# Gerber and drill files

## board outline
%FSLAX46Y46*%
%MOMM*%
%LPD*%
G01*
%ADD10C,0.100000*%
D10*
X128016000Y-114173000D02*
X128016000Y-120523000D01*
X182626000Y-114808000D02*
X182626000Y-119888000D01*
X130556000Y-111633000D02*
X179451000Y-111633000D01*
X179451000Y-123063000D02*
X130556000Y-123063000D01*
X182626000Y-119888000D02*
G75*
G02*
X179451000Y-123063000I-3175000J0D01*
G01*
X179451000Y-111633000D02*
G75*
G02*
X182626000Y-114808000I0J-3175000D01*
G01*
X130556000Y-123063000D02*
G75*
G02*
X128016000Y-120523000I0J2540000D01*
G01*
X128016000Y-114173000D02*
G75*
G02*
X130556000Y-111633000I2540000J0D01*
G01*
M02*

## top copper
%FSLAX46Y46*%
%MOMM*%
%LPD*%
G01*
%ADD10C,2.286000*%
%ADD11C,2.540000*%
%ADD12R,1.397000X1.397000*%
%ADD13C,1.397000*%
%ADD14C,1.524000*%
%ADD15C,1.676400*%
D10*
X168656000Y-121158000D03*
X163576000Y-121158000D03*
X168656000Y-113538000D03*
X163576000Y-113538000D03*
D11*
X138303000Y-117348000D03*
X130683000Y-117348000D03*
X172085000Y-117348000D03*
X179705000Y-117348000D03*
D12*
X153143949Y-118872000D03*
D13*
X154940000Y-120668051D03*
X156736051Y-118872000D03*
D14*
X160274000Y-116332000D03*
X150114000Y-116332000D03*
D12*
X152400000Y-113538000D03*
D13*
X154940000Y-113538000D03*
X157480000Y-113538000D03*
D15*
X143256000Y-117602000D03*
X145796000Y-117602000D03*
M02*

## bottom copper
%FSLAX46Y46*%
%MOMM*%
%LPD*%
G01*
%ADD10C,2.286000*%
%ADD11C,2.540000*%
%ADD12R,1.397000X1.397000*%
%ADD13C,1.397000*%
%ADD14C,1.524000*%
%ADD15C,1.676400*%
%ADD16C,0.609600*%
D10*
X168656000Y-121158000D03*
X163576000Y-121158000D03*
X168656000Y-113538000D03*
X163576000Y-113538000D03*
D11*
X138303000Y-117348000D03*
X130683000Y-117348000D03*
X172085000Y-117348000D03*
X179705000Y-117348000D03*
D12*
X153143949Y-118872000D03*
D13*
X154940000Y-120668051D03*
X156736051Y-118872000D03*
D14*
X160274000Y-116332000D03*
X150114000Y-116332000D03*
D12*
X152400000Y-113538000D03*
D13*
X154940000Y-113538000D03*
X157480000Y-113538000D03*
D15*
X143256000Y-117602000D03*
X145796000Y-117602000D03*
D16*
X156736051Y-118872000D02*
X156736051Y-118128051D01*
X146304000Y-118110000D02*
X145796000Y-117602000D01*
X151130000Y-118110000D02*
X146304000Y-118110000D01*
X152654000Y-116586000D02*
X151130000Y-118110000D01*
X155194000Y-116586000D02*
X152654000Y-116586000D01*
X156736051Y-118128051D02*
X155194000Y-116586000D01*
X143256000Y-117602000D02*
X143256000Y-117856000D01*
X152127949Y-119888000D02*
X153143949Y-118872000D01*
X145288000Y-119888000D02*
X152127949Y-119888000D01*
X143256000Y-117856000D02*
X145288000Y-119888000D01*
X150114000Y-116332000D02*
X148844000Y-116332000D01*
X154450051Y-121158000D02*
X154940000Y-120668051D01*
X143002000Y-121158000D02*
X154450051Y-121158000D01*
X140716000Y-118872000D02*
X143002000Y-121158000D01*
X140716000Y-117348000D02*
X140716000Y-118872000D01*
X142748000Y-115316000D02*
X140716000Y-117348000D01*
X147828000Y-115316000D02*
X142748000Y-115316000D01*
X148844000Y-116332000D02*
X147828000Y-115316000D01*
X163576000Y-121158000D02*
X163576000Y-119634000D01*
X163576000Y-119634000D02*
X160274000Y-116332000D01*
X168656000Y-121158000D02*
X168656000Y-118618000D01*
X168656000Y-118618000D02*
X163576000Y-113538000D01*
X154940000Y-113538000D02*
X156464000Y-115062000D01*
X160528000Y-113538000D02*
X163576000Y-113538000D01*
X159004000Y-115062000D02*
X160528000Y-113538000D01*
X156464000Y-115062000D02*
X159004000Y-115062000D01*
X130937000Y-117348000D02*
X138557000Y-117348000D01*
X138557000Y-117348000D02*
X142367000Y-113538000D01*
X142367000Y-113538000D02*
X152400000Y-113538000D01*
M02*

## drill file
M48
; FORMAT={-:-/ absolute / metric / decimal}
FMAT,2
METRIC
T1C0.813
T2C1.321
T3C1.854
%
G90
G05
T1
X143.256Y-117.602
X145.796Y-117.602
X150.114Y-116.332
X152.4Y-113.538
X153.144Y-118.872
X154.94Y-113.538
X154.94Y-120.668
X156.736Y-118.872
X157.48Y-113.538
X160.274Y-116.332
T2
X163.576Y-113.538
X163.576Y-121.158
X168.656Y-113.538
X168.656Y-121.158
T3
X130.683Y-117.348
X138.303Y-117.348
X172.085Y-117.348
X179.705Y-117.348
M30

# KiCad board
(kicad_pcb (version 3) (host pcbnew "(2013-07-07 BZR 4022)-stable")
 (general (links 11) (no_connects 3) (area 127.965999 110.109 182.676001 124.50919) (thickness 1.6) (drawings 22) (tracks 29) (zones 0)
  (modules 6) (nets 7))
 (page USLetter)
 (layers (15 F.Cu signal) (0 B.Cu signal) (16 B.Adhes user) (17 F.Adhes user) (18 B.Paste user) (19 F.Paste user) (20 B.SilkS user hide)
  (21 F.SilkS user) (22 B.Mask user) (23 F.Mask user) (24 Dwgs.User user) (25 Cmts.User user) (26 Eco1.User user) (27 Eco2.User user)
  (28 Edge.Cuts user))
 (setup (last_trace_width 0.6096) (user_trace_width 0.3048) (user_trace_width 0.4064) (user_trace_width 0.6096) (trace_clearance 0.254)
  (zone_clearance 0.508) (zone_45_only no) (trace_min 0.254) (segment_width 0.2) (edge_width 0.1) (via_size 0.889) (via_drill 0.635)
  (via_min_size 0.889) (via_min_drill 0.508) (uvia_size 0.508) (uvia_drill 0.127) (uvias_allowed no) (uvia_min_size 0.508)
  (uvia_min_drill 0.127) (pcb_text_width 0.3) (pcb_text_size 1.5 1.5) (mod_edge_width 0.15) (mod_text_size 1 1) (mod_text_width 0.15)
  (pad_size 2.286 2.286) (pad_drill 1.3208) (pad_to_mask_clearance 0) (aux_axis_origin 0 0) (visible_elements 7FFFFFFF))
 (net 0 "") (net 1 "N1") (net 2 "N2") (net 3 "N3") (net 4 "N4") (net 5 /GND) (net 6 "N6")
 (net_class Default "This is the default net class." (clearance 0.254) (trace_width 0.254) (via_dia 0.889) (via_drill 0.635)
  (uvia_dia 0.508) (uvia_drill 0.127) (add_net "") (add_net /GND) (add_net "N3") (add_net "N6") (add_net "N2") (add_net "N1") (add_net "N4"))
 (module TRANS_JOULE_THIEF (layer F.Cu) (at 166.116 118.618 180)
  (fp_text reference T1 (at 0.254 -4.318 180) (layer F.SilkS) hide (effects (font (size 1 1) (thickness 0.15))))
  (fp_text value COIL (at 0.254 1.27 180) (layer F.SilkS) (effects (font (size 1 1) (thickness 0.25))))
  (pad 1 thru_hole circle (at -2.54 -2.54 180) (size 2.286 2.286) (drill 1.3208) (layers *.Cu *.Mask F.SilkS) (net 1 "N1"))
  (pad 2 thru_hole circle (at 2.54 -2.54 180) (size 2.286 2.286) (drill 1.3208) (layers *.Cu *.Mask F.SilkS) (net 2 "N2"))
  (pad 3 thru_hole circle (at -2.54 5.08 180) (size 2.286 2.286) (drill 1.3208) (layers *.Cu *.Mask F.SilkS) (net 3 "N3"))
  (pad 4 thru_hole circle (at 2.54 5.08 180) (size 2.286 2.286) (drill 1.3208) (layers *.Cu *.Mask F.SilkS) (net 1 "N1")))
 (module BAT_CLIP (layer F.Cu) (at 155.321 117.348)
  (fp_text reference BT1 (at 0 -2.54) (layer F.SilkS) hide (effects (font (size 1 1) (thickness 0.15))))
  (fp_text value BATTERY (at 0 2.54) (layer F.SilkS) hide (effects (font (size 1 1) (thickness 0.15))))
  (pad 1 thru_hole circle (at -17.018 0) (size 2.54 2.54) (drill 1.8542) (layers *.Cu *.Mask F.SilkS) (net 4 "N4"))
  (pad 1 thru_hole circle (at -24.638 0) (size 2.54 2.54) (drill 1.8542) (layers *.Cu *.Mask F.SilkS) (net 4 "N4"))
  (pad 2 thru_hole circle (at 16.764 0) (size 2.54 2.54) (drill 1.8542) (layers *.Cu *.Mask F.SilkS) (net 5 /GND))
  (pad 2 thru_hole circle (at 24.384 0) (size 2.54 2.54) (drill 1.8542) (layers *.Cu *.Mask F.SilkS) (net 5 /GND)))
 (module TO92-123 (layer F.Cu) (at 154.94 118.872 135)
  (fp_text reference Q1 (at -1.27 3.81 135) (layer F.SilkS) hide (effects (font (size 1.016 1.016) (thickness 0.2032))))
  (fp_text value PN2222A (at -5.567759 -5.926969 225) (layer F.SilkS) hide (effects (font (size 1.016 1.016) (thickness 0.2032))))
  (pad 3 thru_hole rect (at 1.27 -1.27 180) (size 1.397 1.397) (drill 0.8128) (layers *.Cu *.Mask F.SilkS) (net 3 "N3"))
  (pad 2 thru_hole circle (at -1.27 -1.27 135) (size 1.397 1.397) (drill 0.8128) (layers *.Cu *.Mask F.SilkS) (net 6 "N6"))
  (pad 1 thru_hole circle (at -1.27 1.27 135) (size 1.397 1.397) (drill 0.8128) (layers *.Cu *.Mask F.SilkS) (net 5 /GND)))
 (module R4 (layer F.Cu) (at 155.194 116.332 180) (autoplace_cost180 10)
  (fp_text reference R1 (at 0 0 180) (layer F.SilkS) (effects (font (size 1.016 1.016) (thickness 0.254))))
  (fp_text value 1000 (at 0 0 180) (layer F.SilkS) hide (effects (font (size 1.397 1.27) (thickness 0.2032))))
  (pad 1 thru_hole circle (at -5.08 0 180) (size 1.524 1.524) (drill 0.8128) (layers *.Cu *.Mask F.SilkS) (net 2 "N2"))
  (pad 2 thru_hole circle (at 5.08 0 180) (size 1.524 1.524) (drill 0.8128) (layers *.Cu *.Mask F.SilkS) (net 6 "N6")))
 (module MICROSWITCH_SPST (layer F.Cu) (at 154.94 113.538)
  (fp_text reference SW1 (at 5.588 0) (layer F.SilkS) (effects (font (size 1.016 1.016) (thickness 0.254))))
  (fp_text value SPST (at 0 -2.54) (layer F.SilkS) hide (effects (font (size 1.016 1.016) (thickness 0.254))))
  (pad 1 thru_hole rect (at -2.54 0) (size 1.397 1.397) (drill 0.8128) (layers *.Cu *.Mask F.SilkS) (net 4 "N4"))
  (pad 2 thru_hole circle (at 0 0) (size 1.397 1.397) (drill 0.8128) (layers *.Cu *.Mask F.SilkS) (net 1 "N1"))
  (pad 3 thru_hole circle (at 2.54 0) (size 1.397 1.397) (drill 0.8128) (layers *.Cu *.Mask F.SilkS)))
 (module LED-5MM (layer F.Cu) (at 144.526 117.602)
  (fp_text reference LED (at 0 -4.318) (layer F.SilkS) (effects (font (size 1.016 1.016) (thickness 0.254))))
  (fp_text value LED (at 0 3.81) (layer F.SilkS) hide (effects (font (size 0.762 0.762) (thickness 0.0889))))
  (pad 1 thru_hole circle (at -1.27 0) (size 1.6764 1.6764) (drill 0.8128) (layers *.Cu *.Mask F.SilkS) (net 3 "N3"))
  (pad 2 thru_hole circle (at 1.27 0) (size 1.6764 1.6764) (drill 0.8128) (layers *.Cu *.Mask F.SilkS) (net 5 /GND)))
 (gr_line (start 128.016 114.173) (end 128.016 120.523) (angle 90) (layer Edge.Cuts) (width 0.1))
 (gr_line (start 182.626 114.808) (end 182.626 119.888) (angle 90) (layer Edge.Cuts) (width 0.1))
 (gr_line (start 130.556 111.633) (end 179.451 111.633) (angle 90) (layer Edge.Cuts) (width 0.1))
 (gr_line (start 179.451 123.063) (end 130.556 123.063) (angle 90) (layer Edge.Cuts) (width 0.1))
 (gr_arc (start 179.451 119.888) (end 182.626 119.888) (angle 90) (layer Edge.Cuts) (width 0.1))
 (gr_arc (start 179.451 114.808) (end 179.451 111.633) (angle 90) (layer Edge.Cuts) (width 0.1))
 (gr_arc (start 130.556 120.523) (end 130.556 123.063) (angle 90) (layer Edge.Cuts) (width 0.1))
 (gr_arc (start 130.556 114.173) (end 128.016 114.173) (angle 90) (layer Edge.Cuts) (width 0.1))
 (segment (start 156.736051 118.872) (end 156.736051 118.128051) (width 0.6096) (layer B.Cu) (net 5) (status 400000))
 (segment (start 146.304 118.11) (end 145.796 117.602) (width 0.6096) (layer B.Cu) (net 5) (status C00000))
 (segment (start 151.13 118.11) (end 146.304 118.11) (width 0.6096) (layer B.Cu) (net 5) (status 800000))
 (segment (start 152.654 116.586) (end 151.13 118.11) (width 0.6096) (layer B.Cu) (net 5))
 (segment (start 155.194 116.586) (end 152.654 116.586) (width 0.6096) (layer B.Cu) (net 5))
 (segment (start 156.736051 118.128051) (end 155.194 116.586) (width 0.6096) (layer B.Cu) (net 5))
 (segment (start 143.256 117.602) (end 143.256 117.856) (width 0.6096) (layer B.Cu) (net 3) (status C00000))
 (segment (start 152.127949 119.888) (end 153.143949 118.872) (width 0.6096) (layer B.Cu) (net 3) (status 800000))
 (segment (start 145.288 119.888) (end 152.127949 119.888) (width 0.6096) (layer B.Cu) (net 3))
 (segment (start 143.256 117.856) (end 145.288 119.888) (width 0.6096) (layer B.Cu) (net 3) (status 400000))
 (segment (start 150.114 116.332) (end 148.844 116.332) (width 0.6096) (layer B.Cu) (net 6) (status 400000))
 (segment (start 154.450051 121.158) (end 154.94 120.668051) (width 0.6096) (layer B.Cu) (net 6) (status C00000))
 (segment (start 143.002 121.158) (end 154.450051 121.158) (width 0.6096) (layer B.Cu) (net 6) (status 800000))
 (segment (start 140.716 118.872) (end 143.002 121.158) (width 0.6096) (layer B.Cu) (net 6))
 (segment (start 140.716 117.348) (end 140.716 118.872) (width 0.6096) (layer B.Cu) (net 6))
 (segment (start 142.748 115.316) (end 140.716 117.348) (width 0.6096) (layer B.Cu) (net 6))
 (segment (start 147.828 115.316) (end 142.748 115.316) (width 0.6096) (layer B.Cu) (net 6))
 (segment (start 148.844 116.332) (end 147.828 115.316) (width 0.6096) (layer B.Cu) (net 6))
 (segment (start 163.576 121.158) (end 163.576 119.634) (width 0.6096) (layer B.Cu) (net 2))
 (segment (start 163.576 119.634) (end 160.274 116.332) (width 0.6096) (layer B.Cu) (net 2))
 (segment (start 168.656 121.158) (end 168.656 118.618) (width 0.6096) (layer B.Cu) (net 1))
 (segment (start 168.656 118.618) (end 163.576 113.538) (width 0.6096) (layer B.Cu) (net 1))
 (segment (start 154.94 113.538) (end 156.464 115.062) (width 0.6096) (layer B.Cu) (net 1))
 (segment (start 160.528 113.538) (end 163.576 113.538) (width 0.6096) (layer B.Cu) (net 1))
 (segment (start 159.004 115.062) (end 160.528 113.538) (width 0.6096) (layer B.Cu) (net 1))
 (segment (start 156.464 115.062) (end 159.004 115.062) (width 0.6096) (layer B.Cu) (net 1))
 (segment (start 130.937 117.348) (end 138.557 117.348) (width 0.6096) (layer B.Cu) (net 4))
 (segment (start 138.557 117.348) (end 142.367 113.538) (width 0.6096) (layer B.Cu) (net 4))
 (segment (start 142.367 113.538) (end 152.4 113.538) (width 0.6096) (layer B.Cu) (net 4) (status 20)))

